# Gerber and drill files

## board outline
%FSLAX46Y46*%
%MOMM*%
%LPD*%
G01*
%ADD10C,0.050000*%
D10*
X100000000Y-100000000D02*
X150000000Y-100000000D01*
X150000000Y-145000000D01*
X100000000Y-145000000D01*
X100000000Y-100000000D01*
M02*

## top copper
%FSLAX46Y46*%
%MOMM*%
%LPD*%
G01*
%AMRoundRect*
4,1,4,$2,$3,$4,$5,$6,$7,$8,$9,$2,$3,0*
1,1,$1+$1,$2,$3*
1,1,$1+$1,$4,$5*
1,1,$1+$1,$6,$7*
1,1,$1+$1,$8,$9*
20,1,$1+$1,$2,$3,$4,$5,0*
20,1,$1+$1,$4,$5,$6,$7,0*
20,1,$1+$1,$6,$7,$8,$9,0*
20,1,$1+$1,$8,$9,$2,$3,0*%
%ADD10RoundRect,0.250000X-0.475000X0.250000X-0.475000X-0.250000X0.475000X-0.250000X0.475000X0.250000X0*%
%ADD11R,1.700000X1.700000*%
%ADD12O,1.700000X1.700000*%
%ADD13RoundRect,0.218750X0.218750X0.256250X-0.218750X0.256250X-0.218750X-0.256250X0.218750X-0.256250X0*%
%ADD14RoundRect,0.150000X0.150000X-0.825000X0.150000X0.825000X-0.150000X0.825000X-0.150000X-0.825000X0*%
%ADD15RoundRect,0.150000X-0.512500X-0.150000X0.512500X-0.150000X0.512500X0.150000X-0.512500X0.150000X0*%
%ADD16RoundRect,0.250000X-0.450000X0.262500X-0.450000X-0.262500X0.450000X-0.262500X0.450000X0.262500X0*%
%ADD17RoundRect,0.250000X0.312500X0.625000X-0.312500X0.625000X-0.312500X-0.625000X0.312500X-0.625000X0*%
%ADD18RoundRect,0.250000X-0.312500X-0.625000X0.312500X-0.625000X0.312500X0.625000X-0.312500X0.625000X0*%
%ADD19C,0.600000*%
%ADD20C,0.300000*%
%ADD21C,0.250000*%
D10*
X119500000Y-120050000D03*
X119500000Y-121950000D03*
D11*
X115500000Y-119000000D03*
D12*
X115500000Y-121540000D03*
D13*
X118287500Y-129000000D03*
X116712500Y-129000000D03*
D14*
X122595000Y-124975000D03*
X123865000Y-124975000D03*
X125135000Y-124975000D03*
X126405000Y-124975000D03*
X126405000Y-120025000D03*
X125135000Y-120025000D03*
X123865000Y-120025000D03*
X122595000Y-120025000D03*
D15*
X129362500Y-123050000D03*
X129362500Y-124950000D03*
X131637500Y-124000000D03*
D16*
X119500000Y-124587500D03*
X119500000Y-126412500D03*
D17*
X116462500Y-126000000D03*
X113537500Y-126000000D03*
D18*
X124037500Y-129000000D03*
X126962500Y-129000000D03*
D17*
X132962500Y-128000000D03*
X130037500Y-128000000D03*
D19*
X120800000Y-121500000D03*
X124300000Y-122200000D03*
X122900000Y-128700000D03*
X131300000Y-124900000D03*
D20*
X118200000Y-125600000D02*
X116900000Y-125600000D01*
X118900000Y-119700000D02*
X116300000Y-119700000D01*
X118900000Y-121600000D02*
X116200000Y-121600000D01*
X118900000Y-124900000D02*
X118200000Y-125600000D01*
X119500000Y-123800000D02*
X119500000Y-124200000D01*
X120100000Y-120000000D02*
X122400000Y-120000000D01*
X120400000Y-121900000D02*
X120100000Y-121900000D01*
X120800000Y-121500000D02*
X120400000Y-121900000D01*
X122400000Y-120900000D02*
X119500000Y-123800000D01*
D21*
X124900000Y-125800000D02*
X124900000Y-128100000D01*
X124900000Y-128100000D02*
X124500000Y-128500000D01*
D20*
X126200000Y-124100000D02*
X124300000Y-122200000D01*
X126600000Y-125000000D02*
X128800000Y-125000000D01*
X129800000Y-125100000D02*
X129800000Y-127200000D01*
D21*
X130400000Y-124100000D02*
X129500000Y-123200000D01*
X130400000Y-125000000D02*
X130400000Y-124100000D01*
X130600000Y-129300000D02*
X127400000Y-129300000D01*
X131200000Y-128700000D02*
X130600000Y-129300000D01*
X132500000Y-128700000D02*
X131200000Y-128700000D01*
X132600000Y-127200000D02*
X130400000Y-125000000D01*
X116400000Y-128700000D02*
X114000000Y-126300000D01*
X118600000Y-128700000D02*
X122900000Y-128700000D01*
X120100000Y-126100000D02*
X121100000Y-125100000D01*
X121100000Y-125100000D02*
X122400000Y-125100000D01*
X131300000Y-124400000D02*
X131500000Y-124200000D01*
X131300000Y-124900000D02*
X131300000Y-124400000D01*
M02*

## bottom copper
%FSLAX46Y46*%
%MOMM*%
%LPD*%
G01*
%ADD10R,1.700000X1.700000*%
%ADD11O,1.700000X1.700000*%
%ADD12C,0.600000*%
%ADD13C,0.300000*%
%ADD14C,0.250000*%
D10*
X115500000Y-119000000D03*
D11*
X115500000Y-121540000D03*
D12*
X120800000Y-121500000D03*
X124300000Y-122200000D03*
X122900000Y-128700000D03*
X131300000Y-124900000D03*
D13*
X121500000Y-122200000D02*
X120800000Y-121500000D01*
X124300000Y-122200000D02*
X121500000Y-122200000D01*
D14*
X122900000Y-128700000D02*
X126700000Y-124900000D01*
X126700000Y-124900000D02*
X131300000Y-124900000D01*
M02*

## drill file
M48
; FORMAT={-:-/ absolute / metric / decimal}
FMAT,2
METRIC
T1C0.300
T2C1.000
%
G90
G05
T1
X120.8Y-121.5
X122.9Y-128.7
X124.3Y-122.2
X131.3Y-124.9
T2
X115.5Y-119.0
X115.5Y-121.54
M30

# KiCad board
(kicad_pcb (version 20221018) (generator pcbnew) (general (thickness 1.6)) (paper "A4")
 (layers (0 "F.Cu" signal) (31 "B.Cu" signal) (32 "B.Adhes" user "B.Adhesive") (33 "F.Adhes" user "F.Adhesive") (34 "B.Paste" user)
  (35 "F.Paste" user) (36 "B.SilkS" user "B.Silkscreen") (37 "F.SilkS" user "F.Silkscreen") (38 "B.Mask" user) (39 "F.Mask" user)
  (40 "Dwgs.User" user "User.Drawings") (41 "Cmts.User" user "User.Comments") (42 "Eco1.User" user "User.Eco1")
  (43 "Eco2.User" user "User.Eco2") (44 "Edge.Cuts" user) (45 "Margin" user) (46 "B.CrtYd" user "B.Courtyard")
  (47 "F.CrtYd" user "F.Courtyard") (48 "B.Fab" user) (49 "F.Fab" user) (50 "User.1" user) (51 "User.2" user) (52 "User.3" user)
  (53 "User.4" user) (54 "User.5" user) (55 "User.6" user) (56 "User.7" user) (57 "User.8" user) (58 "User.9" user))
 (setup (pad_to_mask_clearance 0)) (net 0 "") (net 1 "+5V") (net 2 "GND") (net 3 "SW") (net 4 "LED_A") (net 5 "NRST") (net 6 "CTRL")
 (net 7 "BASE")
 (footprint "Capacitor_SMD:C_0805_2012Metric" (layer "F.Cu") (at 119.5 121 -90)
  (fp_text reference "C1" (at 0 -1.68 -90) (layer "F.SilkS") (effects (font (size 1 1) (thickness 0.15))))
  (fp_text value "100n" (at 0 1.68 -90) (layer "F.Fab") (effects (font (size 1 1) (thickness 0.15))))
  (pad "1" smd roundrect (at -0.95 0 270) (size 1 1.45) (layers "F.Cu" "F.Paste" "F.Mask") (roundrect_rratio 0.25) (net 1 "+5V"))
  (pad "2" smd roundrect (at 0.95 0 270) (size 1 1.45) (layers "F.Cu" "F.Paste" "F.Mask") (roundrect_rratio 0.25) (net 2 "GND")))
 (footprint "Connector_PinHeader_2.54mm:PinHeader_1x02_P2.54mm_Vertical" (layer "F.Cu") (at 115.5 119)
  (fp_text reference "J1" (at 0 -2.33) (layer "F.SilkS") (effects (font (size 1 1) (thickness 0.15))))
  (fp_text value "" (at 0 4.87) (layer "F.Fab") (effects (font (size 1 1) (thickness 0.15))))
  (pad "1" thru_hole rect (at 0 0) (size 1.7 1.7) (drill 1) (layers "*.Cu" "*.Mask") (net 1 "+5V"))
  (pad "2" thru_hole oval (at 0 2.54) (size 1.7 1.7) (drill 1) (layers "*.Cu" "*.Mask") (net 2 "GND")))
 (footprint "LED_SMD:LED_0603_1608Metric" (layer "F.Cu") (at 117.5 129 180)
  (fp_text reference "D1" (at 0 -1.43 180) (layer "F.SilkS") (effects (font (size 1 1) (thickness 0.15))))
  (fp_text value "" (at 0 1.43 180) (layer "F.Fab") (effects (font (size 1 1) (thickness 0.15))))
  (pad "1" smd roundrect (at -0.7875 0 180) (size 0.875 0.95) (layers "F.Cu" "F.Paste" "F.Mask") (roundrect_rratio 0.25) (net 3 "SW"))
  (pad "2" smd roundrect (at 0.7875 0 180) (size 0.875 0.95) (layers "F.Cu" "F.Paste" "F.Mask") (roundrect_rratio 0.25) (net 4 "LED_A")))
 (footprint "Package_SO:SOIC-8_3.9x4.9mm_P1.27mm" (layer "F.Cu") (at 124.5 122.5 90)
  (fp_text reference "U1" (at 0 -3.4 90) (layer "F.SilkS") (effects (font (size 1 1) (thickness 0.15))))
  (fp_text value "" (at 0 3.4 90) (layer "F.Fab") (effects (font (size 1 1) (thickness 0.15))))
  (pad "1" smd roundrect (at -2.475 -1.905 90) (size 1.95 0.6) (layers "F.Cu" "F.Paste" "F.Mask") (roundrect_rratio 0.25) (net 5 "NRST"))
  (pad "2" smd roundrect (at -2.475 -0.635 90) (size 1.95 0.6) (layers "F.Cu" "F.Paste" "F.Mask") (roundrect_rratio 0.25))
  (pad "3" smd roundrect (at -2.475 0.635 90) (size 1.95 0.6) (layers "F.Cu" "F.Paste" "F.Mask") (roundrect_rratio 0.25) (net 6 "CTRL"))
  (pad "4" smd roundrect (at -2.475 1.905 90) (size 1.95 0.6) (layers "F.Cu" "F.Paste" "F.Mask") (roundrect_rratio 0.25) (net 2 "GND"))
  (pad "5" smd roundrect (at 2.475 1.905 90) (size 1.95 0.6) (layers "F.Cu" "F.Paste" "F.Mask") (roundrect_rratio 0.25))
  (pad "6" smd roundrect (at 2.475 0.635 90) (size 1.95 0.6) (layers "F.Cu" "F.Paste" "F.Mask") (roundrect_rratio 0.25))
  (pad "7" smd roundrect (at 2.475 -0.635 90) (size 1.95 0.6) (layers "F.Cu" "F.Paste" "F.Mask") (roundrect_rratio 0.25))
  (pad "8" smd roundrect (at 2.475 -1.905 90) (size 1.95 0.6) (layers "F.Cu" "F.Paste" "F.Mask") (roundrect_rratio 0.25) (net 1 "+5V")))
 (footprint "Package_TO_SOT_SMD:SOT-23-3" (layer "F.Cu") (at 130.5 124)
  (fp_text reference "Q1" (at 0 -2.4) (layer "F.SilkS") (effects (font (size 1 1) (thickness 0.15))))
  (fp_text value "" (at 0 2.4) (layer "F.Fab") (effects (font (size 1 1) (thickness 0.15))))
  (pad "1" smd roundrect (at -1.1375 -0.95) (size 1.325 0.6) (layers "F.Cu" "F.Paste" "F.Mask") (roundrect_rratio 0.25) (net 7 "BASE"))
  (pad "2" smd roundrect (at -1.1375 0.95) (size 1.325 0.6) (layers "F.Cu" "F.Paste" "F.Mask") (roundrect_rratio 0.25) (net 2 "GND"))
  (pad "3" smd roundrect (at 1.1375 0) (size 1.325 0.6) (layers "F.Cu" "F.Paste" "F.Mask") (roundrect_rratio 0.25) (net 3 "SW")))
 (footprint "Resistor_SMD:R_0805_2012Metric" (layer "F.Cu") (at 119.5 125.5 -90)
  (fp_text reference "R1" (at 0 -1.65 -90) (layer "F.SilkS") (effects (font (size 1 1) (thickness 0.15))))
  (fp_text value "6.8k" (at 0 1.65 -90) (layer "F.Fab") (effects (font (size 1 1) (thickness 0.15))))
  (pad "1" smd roundrect (at -0.9125 0 270) (size 1.025 1.4) (layers "F.Cu" "F.Paste" "F.Mask") (roundrect_rratio 0.243902) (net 1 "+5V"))
  (pad "2" smd roundrect (at 0.9125 0 270) (size 1.025 1.4) (layers "F.Cu" "F.Paste" "F.Mask") (roundrect_rratio 0.243902) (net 5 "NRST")))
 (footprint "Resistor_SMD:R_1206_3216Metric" (layer "F.Cu") (at 115 126 180)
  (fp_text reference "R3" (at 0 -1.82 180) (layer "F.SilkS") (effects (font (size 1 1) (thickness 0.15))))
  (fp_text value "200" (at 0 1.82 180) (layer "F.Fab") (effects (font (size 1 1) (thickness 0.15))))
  (pad "1" smd roundrect (at -1.4625 0 180) (size 1.125 1.75) (layers "F.Cu" "F.Paste" "F.Mask") (roundrect_rratio 0.222222) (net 1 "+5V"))
  (pad "2" smd roundrect (at 1.4625 0 180) (size 1.125 1.75) (layers "F.Cu" "F.Paste" "F.Mask") (roundrect_rratio 0.222222) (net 4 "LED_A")))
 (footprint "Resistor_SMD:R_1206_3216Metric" (layer "F.Cu") (at 125.5 129)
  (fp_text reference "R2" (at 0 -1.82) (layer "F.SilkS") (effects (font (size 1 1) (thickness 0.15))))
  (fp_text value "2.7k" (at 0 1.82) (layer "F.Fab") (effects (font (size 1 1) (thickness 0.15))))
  (pad "1" smd roundrect (at -1.4625 0) (size 1.125 1.75) (layers "F.Cu" "F.Paste" "F.Mask") (roundrect_rratio 0.222222) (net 6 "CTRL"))
  (pad "2" smd roundrect (at 1.4625 0) (size 1.125 1.75) (layers "F.Cu" "F.Paste" "F.Mask") (roundrect_rratio 0.222222) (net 7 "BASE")))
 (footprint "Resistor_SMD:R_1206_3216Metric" (layer "F.Cu") (at 131.5 128 180)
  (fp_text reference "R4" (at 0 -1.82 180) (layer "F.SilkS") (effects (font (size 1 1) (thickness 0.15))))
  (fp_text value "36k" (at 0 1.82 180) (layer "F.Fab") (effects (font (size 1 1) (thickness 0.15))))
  (pad "1" smd roundrect (at -1.4625 0 180) (size 1.125 1.75) (layers "F.Cu" "F.Paste" "F.Mask") (roundrect_rratio 0.222222) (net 7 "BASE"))
  (pad "2" smd roundrect (at 1.4625 0 180) (size 1.125 1.75) (layers "F.Cu" "F.Paste" "F.Mask") (roundrect_rratio 0.222222) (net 2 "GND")))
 (gr_rect (start 100 100) (end 150 145) (stroke (width 0.05) (type default)) (fill none) (layer "Edge.Cuts"))
 (segment (start 118.2 125.6) (end 116.9 125.6) (width 0.3) (layer "F.Cu") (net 1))
 (segment (start 118.9 119.7) (end 116.3 119.7) (width 0.3) (layer "F.Cu") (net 1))
 (segment (start 118.9 121.6) (end 116.2 121.6) (width 0.3) (layer "F.Cu") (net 2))
 (segment (start 118.9 124.9) (end 118.2 125.6) (width 0.3) (layer "F.Cu") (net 1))
 (segment (start 119.5 123.8) (end 119.5 124.2) (width 0.3) (layer "F.Cu") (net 1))
 (segment (start 120.1 120) (end 122.4 120) (width 0.3) (layer "F.Cu") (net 1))
 (segment (start 120.4 121.9) (end 120.1 121.9) (width 0.3) (layer "F.Cu") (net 2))
 (segment (start 120.8 121.5) (end 120.4 121.9) (width 0.3) (layer "F.Cu") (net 2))
 (segment (start 122.4 120.9) (end 119.5 123.8) (width 0.3) (layer "F.Cu") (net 1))
 (segment (start 124.9 125.8) (end 124.9 128.1) (width 0.25) (layer "F.Cu") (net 6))
 (segment (start 124.9 128.1) (end 124.5 128.5) (width 0.25) (layer "F.Cu") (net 6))
 (segment (start 126.2 124.1) (end 124.3 122.2) (width 0.3) (layer "F.Cu") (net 2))
 (segment (start 126.6 125) (end 128.8 125) (width 0.3) (layer "F.Cu") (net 2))
 (segment (start 129.8 125.1) (end 129.8 127.2) (width 0.3) (layer "F.Cu") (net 2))
 (segment (start 130.4 124.1) (end 129.5 123.2) (width 0.25) (layer "F.Cu") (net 7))
 (segment (start 130.4 125) (end 130.4 124.1) (width 0.25) (layer "F.Cu") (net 7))
 (segment (start 130.6 129.3) (end 127.4 129.3) (width 0.25) (layer "F.Cu") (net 7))
 (segment (start 131.2 128.7) (end 130.6 129.3) (width 0.25) (layer "F.Cu") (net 7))
 (segment (start 132.5 128.7) (end 131.2 128.7) (width 0.25) (layer "F.Cu") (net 7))
 (segment (start 132.6 127.2) (end 130.4 125) (width 0.25) (layer "F.Cu") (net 7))
 (via (at 120.8 121.5) (size 0.6) (drill 0.3) (layers "F.Cu" "B.Cu") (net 2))
 (via (at 124.3 122.2) (size 0.6) (drill 0.3) (layers "F.Cu" "B.Cu") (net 2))
 (segment (start 116.4 128.7) (end 114 126.3) (width 0.25) (layer "F.Cu") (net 4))
 (segment (start 118.6 128.7) (end 122.9 128.7) (width 0.25) (layer "F.Cu") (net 3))
 (segment (start 120.1 126.1) (end 121.1 125.1) (width 0.25) (layer "F.Cu") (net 5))
 (segment (start 121.1 125.1) (end 122.4 125.1) (width 0.25) (layer "F.Cu") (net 5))
 (segment (start 121.5 122.2) (end 120.8 121.5) (width 0.3) (layer "B.Cu") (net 2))
 (segment (start 124.3 122.2) (end 121.5 122.2) (width 0.3) (layer "B.Cu") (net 2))
 (segment (start 131.3 124.4) (end 131.5 124.2) (width 0.25) (layer "F.Cu") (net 3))
 (segment (start 131.3 124.9) (end 131.3 124.4) (width 0.25) (layer "F.Cu") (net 3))
 (via (at 122.9 128.7) (size 0.6) (drill 0.3) (layers "F.Cu" "B.Cu") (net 3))
 (via (at 131.3 124.9) (size 0.6) (drill 0.3) (layers "F.Cu" "B.Cu") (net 3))
 (segment (start 122.9 128.7) (end 126.7 124.9) (width 0.25) (layer "B.Cu") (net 3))
 (segment (start 126.7 124.9) (end 131.3 124.9) (width 0.25) (layer "B.Cu") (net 3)))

